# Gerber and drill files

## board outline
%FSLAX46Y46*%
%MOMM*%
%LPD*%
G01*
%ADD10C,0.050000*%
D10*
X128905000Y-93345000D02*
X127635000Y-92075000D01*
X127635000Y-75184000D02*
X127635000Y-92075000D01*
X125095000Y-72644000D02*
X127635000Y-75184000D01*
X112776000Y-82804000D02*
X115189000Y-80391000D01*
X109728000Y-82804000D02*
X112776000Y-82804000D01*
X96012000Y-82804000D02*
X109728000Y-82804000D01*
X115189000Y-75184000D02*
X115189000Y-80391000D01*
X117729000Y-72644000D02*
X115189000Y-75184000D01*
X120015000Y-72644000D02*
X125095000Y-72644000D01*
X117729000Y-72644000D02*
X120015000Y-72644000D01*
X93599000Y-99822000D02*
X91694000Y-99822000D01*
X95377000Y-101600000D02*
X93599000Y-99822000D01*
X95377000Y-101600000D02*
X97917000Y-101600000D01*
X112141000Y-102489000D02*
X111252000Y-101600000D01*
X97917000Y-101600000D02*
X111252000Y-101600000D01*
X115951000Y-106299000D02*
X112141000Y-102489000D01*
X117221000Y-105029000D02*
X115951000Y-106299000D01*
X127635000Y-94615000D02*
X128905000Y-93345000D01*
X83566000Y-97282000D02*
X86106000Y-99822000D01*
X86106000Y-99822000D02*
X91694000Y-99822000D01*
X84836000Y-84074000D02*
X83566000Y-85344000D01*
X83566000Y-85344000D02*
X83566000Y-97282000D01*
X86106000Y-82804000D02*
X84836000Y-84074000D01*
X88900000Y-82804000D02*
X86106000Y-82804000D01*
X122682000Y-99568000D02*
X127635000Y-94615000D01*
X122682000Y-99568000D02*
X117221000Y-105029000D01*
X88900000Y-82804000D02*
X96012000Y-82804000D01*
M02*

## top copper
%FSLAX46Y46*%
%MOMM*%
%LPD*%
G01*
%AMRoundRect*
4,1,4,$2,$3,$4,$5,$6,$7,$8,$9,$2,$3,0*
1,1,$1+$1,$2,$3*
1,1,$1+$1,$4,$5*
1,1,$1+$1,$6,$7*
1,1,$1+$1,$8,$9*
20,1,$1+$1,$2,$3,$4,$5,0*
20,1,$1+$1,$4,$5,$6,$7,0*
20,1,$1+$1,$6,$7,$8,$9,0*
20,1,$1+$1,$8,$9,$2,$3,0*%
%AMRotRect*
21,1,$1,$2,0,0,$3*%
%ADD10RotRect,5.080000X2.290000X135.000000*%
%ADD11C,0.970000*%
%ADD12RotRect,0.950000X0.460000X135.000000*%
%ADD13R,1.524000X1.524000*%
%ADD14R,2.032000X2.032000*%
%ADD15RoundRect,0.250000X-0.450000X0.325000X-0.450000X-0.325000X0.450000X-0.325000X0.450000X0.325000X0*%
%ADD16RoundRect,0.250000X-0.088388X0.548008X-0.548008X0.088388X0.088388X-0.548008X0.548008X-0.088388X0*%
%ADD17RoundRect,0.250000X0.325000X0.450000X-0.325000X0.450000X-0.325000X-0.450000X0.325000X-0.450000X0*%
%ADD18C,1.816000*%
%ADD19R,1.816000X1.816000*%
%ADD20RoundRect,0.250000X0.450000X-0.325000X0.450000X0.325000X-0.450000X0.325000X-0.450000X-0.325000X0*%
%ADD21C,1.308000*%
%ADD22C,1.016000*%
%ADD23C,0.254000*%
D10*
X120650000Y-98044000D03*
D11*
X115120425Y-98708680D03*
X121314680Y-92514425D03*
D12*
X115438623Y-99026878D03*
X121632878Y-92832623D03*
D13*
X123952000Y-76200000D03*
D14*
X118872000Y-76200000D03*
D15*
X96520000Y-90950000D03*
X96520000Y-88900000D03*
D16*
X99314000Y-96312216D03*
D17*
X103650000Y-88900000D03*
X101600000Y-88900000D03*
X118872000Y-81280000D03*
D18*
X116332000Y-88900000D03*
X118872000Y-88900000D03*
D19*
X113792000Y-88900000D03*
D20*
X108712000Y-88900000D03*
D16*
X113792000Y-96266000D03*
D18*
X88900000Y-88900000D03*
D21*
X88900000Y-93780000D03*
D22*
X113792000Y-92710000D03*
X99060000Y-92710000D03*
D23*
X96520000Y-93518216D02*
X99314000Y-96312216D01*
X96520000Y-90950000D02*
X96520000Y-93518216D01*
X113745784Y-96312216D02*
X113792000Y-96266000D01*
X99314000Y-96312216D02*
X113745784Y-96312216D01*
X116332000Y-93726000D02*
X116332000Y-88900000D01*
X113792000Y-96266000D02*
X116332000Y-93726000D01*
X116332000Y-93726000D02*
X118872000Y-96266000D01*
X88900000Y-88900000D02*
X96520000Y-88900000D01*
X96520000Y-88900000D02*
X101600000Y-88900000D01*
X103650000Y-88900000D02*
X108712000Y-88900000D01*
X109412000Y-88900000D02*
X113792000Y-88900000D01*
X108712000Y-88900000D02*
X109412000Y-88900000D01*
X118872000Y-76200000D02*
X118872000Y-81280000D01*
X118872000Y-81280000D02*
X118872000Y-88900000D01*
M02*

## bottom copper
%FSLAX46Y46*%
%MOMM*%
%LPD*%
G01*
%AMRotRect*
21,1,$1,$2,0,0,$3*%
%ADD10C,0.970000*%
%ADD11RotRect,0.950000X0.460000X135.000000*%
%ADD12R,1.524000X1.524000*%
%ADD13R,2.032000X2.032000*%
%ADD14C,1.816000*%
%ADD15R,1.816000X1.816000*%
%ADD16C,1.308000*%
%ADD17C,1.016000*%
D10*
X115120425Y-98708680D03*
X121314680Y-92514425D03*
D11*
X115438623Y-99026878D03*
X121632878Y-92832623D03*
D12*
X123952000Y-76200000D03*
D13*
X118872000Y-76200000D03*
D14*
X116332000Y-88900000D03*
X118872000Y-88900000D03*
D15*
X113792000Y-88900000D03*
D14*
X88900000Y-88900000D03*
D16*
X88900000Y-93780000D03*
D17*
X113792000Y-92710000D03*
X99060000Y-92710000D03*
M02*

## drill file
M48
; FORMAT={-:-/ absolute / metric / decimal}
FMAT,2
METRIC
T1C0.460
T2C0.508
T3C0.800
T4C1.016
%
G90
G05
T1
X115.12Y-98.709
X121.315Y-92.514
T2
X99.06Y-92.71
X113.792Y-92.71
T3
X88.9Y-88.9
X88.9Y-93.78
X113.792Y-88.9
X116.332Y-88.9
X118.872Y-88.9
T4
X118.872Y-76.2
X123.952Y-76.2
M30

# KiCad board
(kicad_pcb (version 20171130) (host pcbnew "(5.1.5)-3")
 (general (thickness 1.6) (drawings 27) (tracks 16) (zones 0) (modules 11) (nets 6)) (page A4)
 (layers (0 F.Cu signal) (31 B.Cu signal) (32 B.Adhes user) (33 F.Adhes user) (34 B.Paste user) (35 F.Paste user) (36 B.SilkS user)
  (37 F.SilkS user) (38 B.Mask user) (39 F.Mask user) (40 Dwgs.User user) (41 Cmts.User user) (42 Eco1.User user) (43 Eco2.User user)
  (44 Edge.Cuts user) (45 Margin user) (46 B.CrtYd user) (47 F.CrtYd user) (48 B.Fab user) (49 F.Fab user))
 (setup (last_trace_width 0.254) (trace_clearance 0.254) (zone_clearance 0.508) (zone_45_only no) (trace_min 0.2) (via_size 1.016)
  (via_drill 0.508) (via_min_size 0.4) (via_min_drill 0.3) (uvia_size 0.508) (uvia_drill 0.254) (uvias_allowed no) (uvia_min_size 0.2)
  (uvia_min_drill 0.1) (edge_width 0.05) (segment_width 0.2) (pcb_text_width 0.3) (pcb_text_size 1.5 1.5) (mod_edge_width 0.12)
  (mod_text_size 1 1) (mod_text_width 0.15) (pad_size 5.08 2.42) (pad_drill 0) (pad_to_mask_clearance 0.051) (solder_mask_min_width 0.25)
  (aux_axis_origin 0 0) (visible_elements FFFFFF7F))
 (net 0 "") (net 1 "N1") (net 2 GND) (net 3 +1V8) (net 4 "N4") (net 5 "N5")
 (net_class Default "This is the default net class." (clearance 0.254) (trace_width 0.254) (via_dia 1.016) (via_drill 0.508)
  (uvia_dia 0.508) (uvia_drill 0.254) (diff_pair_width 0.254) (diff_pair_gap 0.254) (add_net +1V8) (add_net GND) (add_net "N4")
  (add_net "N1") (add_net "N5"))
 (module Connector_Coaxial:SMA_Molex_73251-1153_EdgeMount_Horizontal (layer F.Cu) (at 119.433776 96.827776 135)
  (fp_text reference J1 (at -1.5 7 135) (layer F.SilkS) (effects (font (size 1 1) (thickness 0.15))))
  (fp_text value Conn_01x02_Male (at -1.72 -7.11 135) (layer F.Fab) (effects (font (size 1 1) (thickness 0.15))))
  (pad 1 smd rect (at -1.72 0 135) (size 5.08 2.29) (layers F.Cu F.Paste F.Mask) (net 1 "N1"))
  (pad 2 smd rect (at -1.72 -4.38 135) (size 5.08 2.42) (layers F.Paste F.Mask) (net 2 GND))
  (pad 2 smd rect (at -1.72 4.38 135) (size 5.08 2.42) (layers F.Paste F.Mask) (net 2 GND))
  (pad 2 smd rect (at -1.72 -4.38 135) (size 5.08 2.42) (layers B.Paste B.Mask) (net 2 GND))
  (pad 2 smd rect (at -1.72 4.38 135) (size 5.08 2.42) (layers B.Paste B.Mask) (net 2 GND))
  (pad 2 thru_hole circle (at 1.72 -4.38 135) (size 0.97 0.97) (drill 0.46) (layers *.Cu) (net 2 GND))
  (pad 2 thru_hole circle (at 1.72 4.38 135) (size 0.97 0.97) (drill 0.46) (layers *.Cu) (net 2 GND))
  (pad 2 smd rect (at 1.27 -4.38 135) (size 0.95 0.46) (layers F.Cu) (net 2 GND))
  (pad 2 smd rect (at 1.27 4.38 135) (size 0.95 0.46) (layers F.Cu) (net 2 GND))
  (pad 2 smd rect (at 1.27 -4.38 135) (size 0.95 0.46) (layers B.Cu) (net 2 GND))
  (pad 2 smd rect (at 1.27 4.38 135) (size 0.95 0.46) (layers B.Cu) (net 2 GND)))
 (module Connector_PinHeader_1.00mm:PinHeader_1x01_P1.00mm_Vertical (layer F.Cu) (at 123.952 76.2)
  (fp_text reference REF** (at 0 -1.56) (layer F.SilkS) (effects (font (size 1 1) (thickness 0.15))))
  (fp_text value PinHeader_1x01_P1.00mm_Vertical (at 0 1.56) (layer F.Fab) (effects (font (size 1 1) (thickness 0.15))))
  (pad 1 thru_hole rect (at 0 0) (size 1.524 1.524) (drill 1.016) (layers *.Mask B.Cu) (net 2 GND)))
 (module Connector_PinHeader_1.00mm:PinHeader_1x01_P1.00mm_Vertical (layer F.Cu) (at 118.872 76.2)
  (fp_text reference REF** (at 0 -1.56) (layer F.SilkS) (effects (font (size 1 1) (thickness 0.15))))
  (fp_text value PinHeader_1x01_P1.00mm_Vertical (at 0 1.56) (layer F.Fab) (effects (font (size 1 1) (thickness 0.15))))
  (pad 1 thru_hole rect (at 0 0) (size 2.032 2.032) (drill 1.016) (layers *.Cu *.Mask) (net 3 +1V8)))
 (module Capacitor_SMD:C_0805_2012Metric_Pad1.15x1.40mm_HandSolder (layer F.Cu) (at 96.52 89.925 270)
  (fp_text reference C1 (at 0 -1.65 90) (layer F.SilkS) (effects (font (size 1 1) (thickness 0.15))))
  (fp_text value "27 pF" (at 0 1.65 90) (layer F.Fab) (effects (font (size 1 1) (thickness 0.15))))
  (pad 2 smd roundrect (at 1.025 0 270) (size 1.15 1.4) (layers F.Cu F.Paste F.Mask) (roundrect_rratio 0.217391) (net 1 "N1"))
  (pad 1 smd roundrect (at -1.025 0 270) (size 1.15 1.4) (layers F.Cu F.Paste F.Mask) (roundrect_rratio 0.217391) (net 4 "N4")))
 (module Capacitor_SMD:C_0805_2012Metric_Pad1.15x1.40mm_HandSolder (layer F.Cu) (at 98.589216 97.037 225)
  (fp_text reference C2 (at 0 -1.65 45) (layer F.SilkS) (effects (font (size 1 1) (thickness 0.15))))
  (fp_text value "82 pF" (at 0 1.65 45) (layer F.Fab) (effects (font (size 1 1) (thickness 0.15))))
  (pad 1 smd roundrect (at -1.025 0 225) (size 1.15 1.4) (layers F.Cu F.Paste F.Mask) (roundrect_rratio 0.217391) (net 1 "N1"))
  (pad 2 smd roundrect (at 1.025 0 225) (size 1.15 1.4) (layers F.Paste F.Mask) (roundrect_rratio 0.217) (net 2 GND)))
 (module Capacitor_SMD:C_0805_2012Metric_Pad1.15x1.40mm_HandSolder (layer F.Cu) (at 102.625 88.9 180)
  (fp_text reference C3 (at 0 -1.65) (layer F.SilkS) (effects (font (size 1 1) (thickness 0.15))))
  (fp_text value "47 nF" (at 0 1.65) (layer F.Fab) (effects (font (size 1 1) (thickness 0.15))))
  (pad 1 smd roundrect (at -1.025 0 180) (size 1.15 1.4) (layers F.Cu F.Paste F.Mask) (roundrect_rratio 0.217391) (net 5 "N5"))
  (pad 2 smd roundrect (at 1.025 0 180) (size 1.15 1.4) (layers F.Cu F.Paste F.Mask) (roundrect_rratio 0.217391) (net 4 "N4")))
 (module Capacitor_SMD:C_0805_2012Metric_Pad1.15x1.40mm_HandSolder (layer F.Cu) (at 119.897 81.28 180)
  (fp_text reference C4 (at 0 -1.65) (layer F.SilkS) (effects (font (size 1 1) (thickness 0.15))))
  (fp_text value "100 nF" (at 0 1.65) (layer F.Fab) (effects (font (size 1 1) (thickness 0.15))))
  (pad 2 smd roundrect (at 1.025 0 180) (size 1.15 1.4) (layers F.Cu F.Paste F.Mask) (roundrect_rratio 0.217391) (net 3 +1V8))
  (pad 1 smd roundrect (at -1.025 0 180) (size 1.15 1.4) (layers F.Paste F.Mask) (roundrect_rratio 0.217) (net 2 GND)))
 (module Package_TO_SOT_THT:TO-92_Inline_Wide (layer F.Cu) (at 113.792 88.9)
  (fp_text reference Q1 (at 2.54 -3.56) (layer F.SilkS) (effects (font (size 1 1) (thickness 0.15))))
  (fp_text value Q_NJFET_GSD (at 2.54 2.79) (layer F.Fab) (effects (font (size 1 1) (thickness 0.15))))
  (pad 2 thru_hole circle (at 2.54 0 90) (size 1.816 1.816) (drill 0.8) (layers *.Cu *.Mask) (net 1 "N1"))
  (pad 3 thru_hole circle (at 5.08 0 90) (size 1.816 1.816) (drill 0.8) (layers *.Cu *.Mask) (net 3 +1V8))
  (pad 1 thru_hole rect (at 0 0 90) (size 1.816 1.816) (drill 0.8) (layers *.Cu *.Mask) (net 5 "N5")))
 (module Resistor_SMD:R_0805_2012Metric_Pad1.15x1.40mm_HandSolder (layer F.Cu) (at 108.712 87.875 90)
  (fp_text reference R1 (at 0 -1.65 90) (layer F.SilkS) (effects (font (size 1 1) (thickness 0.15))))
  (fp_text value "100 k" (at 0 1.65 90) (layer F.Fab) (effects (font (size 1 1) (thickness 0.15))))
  (pad 1 smd roundrect (at -1.025 0 90) (size 1.15 1.4) (layers F.Cu F.Paste F.Mask) (roundrect_rratio 0.217391) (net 5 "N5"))
  (pad 2 smd roundrect (at 1.025 0 90) (size 1.15 1.4) (layers F.Paste F.Mask) (roundrect_rratio 0.217) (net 2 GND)))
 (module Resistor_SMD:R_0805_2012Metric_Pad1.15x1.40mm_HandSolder (layer F.Cu) (at 113.067216 96.990784 225)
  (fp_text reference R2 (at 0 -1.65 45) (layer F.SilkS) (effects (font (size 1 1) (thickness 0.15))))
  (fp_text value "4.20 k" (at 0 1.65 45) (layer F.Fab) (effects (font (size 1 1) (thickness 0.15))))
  (pad 2 smd roundrect (at 1.025 0 225) (size 1.15 1.4) (layers F.Paste F.Mask) (roundrect_rratio 0.217) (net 2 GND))
  (pad 1 smd roundrect (at -1.025 0 225) (size 1.15 1.4) (layers F.Cu F.Paste F.Mask) (roundrect_rratio 0.217391) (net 1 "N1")))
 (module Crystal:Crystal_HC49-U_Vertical (layer F.Cu) (at 88.9 88.9 270)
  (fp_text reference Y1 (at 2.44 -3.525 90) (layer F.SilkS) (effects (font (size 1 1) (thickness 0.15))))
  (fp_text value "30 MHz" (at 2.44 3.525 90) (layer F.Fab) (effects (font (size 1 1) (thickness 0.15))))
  (pad 1 thru_hole circle (at 0 0 270) (size 1.816 1.816) (drill 0.8) (layers *.Cu *.Mask) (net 4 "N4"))
  (pad 2 thru_hole circle (at 4.88 0 270) (size 1.308 1.308) (drill 0.8) (layers *.Mask B.Cu) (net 2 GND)))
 (gr_line (start 128.905 93.345) (end 127.635 92.075) (layer Edge.Cuts) (width 0.05))
 (gr_line (start 127.635 75.184) (end 127.635 92.075) (layer Edge.Cuts) (width 0.05))
 (gr_line (start 125.095 72.644) (end 127.635 75.184) (layer Edge.Cuts) (width 0.05))
 (gr_line (start 112.776 82.804) (end 115.189 80.391) (layer Edge.Cuts) (width 0.05))
 (gr_line (start 109.728 82.804) (end 112.776 82.804) (layer Edge.Cuts) (width 0.05))
 (gr_line (start 96.012 82.804) (end 109.728 82.804) (layer Edge.Cuts) (width 0.05))
 (gr_line (start 115.189 75.184) (end 115.189 80.391) (layer Edge.Cuts) (width 0.05))
 (gr_line (start 117.729 72.644) (end 115.189 75.184) (layer Edge.Cuts) (width 0.05))
 (gr_line (start 120.015 72.644) (end 125.095 72.644) (layer Edge.Cuts) (width 0.05))
 (gr_line (start 117.729 72.644) (end 120.015 72.644) (layer Edge.Cuts) (width 0.05))
 (gr_line (start 93.599 99.822) (end 91.694 99.822) (layer Edge.Cuts) (width 0.05))
 (gr_line (start 95.377 101.6) (end 93.599 99.822) (layer Edge.Cuts) (width 0.05))
 (gr_line (start 95.377 101.6) (end 97.917 101.6) (layer Edge.Cuts) (width 0.05))
 (gr_line (start 112.141 102.489) (end 111.252 101.6) (layer Edge.Cuts) (width 0.05))
 (gr_line (start 97.917 101.6) (end 111.252 101.6) (layer Edge.Cuts) (width 0.05))
 (gr_line (start 115.951 106.299) (end 112.141 102.489) (layer Edge.Cuts) (width 0.05))
 (gr_line (start 117.221 105.029) (end 115.951 106.299) (layer Edge.Cuts) (width 0.05))
 (gr_line (start 127.635 94.615) (end 128.905 93.345) (layer Edge.Cuts) (width 0.05))
 (gr_line (start 83.566 97.282) (end 86.106 99.822) (layer Edge.Cuts) (width 0.05))
 (gr_line (start 86.106 99.822) (end 91.694 99.822) (layer Edge.Cuts) (width 0.05))
 (gr_line (start 84.836 84.074) (end 83.566 85.344) (layer Edge.Cuts) (width 0.05))
 (gr_line (start 83.566 85.344) (end 83.566 97.282) (layer Edge.Cuts) (width 0.05))
 (gr_line (start 86.106 82.804) (end 84.836 84.074) (layer Edge.Cuts) (width 0.05))
 (gr_line (start 88.9 82.804) (end 86.106 82.804) (layer Edge.Cuts) (width 0.05))
 (gr_line (start 122.682 99.568) (end 127.635 94.615) (layer Edge.Cuts) (width 0.05))
 (gr_line (start 122.682 99.568) (end 117.221 105.029) (layer Edge.Cuts) (width 0.05))
 (gr_line (start 88.9 82.804) (end 96.012 82.804) (layer Edge.Cuts) (width 0.05))
 (via (at 113.792 92.71) (size 1.016) (drill 0.508) (layers F.Cu B.Cu) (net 2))
 (via (at 99.06 92.71) (size 1.016) (drill 0.508) (layers F.Cu B.Cu) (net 2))
 (segment (start 96.52 93.518216) (end 99.314 96.312216) (width 0.254) (layer F.Cu) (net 1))
 (segment (start 96.52 90.95) (end 96.52 93.518216) (width 0.254) (layer F.Cu) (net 1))
 (segment (start 113.745784 96.312216) (end 113.792 96.266) (width 0.254) (layer F.Cu) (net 1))
 (segment (start 99.314 96.312216) (end 113.745784 96.312216) (width 0.254) (layer F.Cu) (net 1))
 (segment (start 116.332 93.726) (end 116.332 88.9) (width 0.254) (layer F.Cu) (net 1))
 (segment (start 113.792 96.266) (end 116.332 93.726) (width 0.254) (layer F.Cu) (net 1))
 (segment (start 116.332 93.726) (end 118.872 96.266) (width 0.254) (layer F.Cu) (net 1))
 (segment (start 88.9 88.9) (end 96.52 88.9) (width 0.254) (layer F.Cu) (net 4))
 (segment (start 96.52 88.9) (end 101.6 88.9) (width 0.254) (layer F.Cu) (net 4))
 (segment (start 103.65 88.9) (end 108.712 88.9) (width 0.254) (layer F.Cu) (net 5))
 (segment (start 109.412 88.9) (end 113.792 88.9) (width 0.254) (layer F.Cu) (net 5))
 (segment (start 108.712 88.9) (end 109.412 88.9) (width 0.254) (layer F.Cu) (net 5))
 (segment (start 118.872 76.2) (end 118.872 81.28) (width 0.254) (layer F.Cu) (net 3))
 (segment (start 118.872 81.28) (end 118.872 88.9) (width 0.254) (layer F.Cu) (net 3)))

